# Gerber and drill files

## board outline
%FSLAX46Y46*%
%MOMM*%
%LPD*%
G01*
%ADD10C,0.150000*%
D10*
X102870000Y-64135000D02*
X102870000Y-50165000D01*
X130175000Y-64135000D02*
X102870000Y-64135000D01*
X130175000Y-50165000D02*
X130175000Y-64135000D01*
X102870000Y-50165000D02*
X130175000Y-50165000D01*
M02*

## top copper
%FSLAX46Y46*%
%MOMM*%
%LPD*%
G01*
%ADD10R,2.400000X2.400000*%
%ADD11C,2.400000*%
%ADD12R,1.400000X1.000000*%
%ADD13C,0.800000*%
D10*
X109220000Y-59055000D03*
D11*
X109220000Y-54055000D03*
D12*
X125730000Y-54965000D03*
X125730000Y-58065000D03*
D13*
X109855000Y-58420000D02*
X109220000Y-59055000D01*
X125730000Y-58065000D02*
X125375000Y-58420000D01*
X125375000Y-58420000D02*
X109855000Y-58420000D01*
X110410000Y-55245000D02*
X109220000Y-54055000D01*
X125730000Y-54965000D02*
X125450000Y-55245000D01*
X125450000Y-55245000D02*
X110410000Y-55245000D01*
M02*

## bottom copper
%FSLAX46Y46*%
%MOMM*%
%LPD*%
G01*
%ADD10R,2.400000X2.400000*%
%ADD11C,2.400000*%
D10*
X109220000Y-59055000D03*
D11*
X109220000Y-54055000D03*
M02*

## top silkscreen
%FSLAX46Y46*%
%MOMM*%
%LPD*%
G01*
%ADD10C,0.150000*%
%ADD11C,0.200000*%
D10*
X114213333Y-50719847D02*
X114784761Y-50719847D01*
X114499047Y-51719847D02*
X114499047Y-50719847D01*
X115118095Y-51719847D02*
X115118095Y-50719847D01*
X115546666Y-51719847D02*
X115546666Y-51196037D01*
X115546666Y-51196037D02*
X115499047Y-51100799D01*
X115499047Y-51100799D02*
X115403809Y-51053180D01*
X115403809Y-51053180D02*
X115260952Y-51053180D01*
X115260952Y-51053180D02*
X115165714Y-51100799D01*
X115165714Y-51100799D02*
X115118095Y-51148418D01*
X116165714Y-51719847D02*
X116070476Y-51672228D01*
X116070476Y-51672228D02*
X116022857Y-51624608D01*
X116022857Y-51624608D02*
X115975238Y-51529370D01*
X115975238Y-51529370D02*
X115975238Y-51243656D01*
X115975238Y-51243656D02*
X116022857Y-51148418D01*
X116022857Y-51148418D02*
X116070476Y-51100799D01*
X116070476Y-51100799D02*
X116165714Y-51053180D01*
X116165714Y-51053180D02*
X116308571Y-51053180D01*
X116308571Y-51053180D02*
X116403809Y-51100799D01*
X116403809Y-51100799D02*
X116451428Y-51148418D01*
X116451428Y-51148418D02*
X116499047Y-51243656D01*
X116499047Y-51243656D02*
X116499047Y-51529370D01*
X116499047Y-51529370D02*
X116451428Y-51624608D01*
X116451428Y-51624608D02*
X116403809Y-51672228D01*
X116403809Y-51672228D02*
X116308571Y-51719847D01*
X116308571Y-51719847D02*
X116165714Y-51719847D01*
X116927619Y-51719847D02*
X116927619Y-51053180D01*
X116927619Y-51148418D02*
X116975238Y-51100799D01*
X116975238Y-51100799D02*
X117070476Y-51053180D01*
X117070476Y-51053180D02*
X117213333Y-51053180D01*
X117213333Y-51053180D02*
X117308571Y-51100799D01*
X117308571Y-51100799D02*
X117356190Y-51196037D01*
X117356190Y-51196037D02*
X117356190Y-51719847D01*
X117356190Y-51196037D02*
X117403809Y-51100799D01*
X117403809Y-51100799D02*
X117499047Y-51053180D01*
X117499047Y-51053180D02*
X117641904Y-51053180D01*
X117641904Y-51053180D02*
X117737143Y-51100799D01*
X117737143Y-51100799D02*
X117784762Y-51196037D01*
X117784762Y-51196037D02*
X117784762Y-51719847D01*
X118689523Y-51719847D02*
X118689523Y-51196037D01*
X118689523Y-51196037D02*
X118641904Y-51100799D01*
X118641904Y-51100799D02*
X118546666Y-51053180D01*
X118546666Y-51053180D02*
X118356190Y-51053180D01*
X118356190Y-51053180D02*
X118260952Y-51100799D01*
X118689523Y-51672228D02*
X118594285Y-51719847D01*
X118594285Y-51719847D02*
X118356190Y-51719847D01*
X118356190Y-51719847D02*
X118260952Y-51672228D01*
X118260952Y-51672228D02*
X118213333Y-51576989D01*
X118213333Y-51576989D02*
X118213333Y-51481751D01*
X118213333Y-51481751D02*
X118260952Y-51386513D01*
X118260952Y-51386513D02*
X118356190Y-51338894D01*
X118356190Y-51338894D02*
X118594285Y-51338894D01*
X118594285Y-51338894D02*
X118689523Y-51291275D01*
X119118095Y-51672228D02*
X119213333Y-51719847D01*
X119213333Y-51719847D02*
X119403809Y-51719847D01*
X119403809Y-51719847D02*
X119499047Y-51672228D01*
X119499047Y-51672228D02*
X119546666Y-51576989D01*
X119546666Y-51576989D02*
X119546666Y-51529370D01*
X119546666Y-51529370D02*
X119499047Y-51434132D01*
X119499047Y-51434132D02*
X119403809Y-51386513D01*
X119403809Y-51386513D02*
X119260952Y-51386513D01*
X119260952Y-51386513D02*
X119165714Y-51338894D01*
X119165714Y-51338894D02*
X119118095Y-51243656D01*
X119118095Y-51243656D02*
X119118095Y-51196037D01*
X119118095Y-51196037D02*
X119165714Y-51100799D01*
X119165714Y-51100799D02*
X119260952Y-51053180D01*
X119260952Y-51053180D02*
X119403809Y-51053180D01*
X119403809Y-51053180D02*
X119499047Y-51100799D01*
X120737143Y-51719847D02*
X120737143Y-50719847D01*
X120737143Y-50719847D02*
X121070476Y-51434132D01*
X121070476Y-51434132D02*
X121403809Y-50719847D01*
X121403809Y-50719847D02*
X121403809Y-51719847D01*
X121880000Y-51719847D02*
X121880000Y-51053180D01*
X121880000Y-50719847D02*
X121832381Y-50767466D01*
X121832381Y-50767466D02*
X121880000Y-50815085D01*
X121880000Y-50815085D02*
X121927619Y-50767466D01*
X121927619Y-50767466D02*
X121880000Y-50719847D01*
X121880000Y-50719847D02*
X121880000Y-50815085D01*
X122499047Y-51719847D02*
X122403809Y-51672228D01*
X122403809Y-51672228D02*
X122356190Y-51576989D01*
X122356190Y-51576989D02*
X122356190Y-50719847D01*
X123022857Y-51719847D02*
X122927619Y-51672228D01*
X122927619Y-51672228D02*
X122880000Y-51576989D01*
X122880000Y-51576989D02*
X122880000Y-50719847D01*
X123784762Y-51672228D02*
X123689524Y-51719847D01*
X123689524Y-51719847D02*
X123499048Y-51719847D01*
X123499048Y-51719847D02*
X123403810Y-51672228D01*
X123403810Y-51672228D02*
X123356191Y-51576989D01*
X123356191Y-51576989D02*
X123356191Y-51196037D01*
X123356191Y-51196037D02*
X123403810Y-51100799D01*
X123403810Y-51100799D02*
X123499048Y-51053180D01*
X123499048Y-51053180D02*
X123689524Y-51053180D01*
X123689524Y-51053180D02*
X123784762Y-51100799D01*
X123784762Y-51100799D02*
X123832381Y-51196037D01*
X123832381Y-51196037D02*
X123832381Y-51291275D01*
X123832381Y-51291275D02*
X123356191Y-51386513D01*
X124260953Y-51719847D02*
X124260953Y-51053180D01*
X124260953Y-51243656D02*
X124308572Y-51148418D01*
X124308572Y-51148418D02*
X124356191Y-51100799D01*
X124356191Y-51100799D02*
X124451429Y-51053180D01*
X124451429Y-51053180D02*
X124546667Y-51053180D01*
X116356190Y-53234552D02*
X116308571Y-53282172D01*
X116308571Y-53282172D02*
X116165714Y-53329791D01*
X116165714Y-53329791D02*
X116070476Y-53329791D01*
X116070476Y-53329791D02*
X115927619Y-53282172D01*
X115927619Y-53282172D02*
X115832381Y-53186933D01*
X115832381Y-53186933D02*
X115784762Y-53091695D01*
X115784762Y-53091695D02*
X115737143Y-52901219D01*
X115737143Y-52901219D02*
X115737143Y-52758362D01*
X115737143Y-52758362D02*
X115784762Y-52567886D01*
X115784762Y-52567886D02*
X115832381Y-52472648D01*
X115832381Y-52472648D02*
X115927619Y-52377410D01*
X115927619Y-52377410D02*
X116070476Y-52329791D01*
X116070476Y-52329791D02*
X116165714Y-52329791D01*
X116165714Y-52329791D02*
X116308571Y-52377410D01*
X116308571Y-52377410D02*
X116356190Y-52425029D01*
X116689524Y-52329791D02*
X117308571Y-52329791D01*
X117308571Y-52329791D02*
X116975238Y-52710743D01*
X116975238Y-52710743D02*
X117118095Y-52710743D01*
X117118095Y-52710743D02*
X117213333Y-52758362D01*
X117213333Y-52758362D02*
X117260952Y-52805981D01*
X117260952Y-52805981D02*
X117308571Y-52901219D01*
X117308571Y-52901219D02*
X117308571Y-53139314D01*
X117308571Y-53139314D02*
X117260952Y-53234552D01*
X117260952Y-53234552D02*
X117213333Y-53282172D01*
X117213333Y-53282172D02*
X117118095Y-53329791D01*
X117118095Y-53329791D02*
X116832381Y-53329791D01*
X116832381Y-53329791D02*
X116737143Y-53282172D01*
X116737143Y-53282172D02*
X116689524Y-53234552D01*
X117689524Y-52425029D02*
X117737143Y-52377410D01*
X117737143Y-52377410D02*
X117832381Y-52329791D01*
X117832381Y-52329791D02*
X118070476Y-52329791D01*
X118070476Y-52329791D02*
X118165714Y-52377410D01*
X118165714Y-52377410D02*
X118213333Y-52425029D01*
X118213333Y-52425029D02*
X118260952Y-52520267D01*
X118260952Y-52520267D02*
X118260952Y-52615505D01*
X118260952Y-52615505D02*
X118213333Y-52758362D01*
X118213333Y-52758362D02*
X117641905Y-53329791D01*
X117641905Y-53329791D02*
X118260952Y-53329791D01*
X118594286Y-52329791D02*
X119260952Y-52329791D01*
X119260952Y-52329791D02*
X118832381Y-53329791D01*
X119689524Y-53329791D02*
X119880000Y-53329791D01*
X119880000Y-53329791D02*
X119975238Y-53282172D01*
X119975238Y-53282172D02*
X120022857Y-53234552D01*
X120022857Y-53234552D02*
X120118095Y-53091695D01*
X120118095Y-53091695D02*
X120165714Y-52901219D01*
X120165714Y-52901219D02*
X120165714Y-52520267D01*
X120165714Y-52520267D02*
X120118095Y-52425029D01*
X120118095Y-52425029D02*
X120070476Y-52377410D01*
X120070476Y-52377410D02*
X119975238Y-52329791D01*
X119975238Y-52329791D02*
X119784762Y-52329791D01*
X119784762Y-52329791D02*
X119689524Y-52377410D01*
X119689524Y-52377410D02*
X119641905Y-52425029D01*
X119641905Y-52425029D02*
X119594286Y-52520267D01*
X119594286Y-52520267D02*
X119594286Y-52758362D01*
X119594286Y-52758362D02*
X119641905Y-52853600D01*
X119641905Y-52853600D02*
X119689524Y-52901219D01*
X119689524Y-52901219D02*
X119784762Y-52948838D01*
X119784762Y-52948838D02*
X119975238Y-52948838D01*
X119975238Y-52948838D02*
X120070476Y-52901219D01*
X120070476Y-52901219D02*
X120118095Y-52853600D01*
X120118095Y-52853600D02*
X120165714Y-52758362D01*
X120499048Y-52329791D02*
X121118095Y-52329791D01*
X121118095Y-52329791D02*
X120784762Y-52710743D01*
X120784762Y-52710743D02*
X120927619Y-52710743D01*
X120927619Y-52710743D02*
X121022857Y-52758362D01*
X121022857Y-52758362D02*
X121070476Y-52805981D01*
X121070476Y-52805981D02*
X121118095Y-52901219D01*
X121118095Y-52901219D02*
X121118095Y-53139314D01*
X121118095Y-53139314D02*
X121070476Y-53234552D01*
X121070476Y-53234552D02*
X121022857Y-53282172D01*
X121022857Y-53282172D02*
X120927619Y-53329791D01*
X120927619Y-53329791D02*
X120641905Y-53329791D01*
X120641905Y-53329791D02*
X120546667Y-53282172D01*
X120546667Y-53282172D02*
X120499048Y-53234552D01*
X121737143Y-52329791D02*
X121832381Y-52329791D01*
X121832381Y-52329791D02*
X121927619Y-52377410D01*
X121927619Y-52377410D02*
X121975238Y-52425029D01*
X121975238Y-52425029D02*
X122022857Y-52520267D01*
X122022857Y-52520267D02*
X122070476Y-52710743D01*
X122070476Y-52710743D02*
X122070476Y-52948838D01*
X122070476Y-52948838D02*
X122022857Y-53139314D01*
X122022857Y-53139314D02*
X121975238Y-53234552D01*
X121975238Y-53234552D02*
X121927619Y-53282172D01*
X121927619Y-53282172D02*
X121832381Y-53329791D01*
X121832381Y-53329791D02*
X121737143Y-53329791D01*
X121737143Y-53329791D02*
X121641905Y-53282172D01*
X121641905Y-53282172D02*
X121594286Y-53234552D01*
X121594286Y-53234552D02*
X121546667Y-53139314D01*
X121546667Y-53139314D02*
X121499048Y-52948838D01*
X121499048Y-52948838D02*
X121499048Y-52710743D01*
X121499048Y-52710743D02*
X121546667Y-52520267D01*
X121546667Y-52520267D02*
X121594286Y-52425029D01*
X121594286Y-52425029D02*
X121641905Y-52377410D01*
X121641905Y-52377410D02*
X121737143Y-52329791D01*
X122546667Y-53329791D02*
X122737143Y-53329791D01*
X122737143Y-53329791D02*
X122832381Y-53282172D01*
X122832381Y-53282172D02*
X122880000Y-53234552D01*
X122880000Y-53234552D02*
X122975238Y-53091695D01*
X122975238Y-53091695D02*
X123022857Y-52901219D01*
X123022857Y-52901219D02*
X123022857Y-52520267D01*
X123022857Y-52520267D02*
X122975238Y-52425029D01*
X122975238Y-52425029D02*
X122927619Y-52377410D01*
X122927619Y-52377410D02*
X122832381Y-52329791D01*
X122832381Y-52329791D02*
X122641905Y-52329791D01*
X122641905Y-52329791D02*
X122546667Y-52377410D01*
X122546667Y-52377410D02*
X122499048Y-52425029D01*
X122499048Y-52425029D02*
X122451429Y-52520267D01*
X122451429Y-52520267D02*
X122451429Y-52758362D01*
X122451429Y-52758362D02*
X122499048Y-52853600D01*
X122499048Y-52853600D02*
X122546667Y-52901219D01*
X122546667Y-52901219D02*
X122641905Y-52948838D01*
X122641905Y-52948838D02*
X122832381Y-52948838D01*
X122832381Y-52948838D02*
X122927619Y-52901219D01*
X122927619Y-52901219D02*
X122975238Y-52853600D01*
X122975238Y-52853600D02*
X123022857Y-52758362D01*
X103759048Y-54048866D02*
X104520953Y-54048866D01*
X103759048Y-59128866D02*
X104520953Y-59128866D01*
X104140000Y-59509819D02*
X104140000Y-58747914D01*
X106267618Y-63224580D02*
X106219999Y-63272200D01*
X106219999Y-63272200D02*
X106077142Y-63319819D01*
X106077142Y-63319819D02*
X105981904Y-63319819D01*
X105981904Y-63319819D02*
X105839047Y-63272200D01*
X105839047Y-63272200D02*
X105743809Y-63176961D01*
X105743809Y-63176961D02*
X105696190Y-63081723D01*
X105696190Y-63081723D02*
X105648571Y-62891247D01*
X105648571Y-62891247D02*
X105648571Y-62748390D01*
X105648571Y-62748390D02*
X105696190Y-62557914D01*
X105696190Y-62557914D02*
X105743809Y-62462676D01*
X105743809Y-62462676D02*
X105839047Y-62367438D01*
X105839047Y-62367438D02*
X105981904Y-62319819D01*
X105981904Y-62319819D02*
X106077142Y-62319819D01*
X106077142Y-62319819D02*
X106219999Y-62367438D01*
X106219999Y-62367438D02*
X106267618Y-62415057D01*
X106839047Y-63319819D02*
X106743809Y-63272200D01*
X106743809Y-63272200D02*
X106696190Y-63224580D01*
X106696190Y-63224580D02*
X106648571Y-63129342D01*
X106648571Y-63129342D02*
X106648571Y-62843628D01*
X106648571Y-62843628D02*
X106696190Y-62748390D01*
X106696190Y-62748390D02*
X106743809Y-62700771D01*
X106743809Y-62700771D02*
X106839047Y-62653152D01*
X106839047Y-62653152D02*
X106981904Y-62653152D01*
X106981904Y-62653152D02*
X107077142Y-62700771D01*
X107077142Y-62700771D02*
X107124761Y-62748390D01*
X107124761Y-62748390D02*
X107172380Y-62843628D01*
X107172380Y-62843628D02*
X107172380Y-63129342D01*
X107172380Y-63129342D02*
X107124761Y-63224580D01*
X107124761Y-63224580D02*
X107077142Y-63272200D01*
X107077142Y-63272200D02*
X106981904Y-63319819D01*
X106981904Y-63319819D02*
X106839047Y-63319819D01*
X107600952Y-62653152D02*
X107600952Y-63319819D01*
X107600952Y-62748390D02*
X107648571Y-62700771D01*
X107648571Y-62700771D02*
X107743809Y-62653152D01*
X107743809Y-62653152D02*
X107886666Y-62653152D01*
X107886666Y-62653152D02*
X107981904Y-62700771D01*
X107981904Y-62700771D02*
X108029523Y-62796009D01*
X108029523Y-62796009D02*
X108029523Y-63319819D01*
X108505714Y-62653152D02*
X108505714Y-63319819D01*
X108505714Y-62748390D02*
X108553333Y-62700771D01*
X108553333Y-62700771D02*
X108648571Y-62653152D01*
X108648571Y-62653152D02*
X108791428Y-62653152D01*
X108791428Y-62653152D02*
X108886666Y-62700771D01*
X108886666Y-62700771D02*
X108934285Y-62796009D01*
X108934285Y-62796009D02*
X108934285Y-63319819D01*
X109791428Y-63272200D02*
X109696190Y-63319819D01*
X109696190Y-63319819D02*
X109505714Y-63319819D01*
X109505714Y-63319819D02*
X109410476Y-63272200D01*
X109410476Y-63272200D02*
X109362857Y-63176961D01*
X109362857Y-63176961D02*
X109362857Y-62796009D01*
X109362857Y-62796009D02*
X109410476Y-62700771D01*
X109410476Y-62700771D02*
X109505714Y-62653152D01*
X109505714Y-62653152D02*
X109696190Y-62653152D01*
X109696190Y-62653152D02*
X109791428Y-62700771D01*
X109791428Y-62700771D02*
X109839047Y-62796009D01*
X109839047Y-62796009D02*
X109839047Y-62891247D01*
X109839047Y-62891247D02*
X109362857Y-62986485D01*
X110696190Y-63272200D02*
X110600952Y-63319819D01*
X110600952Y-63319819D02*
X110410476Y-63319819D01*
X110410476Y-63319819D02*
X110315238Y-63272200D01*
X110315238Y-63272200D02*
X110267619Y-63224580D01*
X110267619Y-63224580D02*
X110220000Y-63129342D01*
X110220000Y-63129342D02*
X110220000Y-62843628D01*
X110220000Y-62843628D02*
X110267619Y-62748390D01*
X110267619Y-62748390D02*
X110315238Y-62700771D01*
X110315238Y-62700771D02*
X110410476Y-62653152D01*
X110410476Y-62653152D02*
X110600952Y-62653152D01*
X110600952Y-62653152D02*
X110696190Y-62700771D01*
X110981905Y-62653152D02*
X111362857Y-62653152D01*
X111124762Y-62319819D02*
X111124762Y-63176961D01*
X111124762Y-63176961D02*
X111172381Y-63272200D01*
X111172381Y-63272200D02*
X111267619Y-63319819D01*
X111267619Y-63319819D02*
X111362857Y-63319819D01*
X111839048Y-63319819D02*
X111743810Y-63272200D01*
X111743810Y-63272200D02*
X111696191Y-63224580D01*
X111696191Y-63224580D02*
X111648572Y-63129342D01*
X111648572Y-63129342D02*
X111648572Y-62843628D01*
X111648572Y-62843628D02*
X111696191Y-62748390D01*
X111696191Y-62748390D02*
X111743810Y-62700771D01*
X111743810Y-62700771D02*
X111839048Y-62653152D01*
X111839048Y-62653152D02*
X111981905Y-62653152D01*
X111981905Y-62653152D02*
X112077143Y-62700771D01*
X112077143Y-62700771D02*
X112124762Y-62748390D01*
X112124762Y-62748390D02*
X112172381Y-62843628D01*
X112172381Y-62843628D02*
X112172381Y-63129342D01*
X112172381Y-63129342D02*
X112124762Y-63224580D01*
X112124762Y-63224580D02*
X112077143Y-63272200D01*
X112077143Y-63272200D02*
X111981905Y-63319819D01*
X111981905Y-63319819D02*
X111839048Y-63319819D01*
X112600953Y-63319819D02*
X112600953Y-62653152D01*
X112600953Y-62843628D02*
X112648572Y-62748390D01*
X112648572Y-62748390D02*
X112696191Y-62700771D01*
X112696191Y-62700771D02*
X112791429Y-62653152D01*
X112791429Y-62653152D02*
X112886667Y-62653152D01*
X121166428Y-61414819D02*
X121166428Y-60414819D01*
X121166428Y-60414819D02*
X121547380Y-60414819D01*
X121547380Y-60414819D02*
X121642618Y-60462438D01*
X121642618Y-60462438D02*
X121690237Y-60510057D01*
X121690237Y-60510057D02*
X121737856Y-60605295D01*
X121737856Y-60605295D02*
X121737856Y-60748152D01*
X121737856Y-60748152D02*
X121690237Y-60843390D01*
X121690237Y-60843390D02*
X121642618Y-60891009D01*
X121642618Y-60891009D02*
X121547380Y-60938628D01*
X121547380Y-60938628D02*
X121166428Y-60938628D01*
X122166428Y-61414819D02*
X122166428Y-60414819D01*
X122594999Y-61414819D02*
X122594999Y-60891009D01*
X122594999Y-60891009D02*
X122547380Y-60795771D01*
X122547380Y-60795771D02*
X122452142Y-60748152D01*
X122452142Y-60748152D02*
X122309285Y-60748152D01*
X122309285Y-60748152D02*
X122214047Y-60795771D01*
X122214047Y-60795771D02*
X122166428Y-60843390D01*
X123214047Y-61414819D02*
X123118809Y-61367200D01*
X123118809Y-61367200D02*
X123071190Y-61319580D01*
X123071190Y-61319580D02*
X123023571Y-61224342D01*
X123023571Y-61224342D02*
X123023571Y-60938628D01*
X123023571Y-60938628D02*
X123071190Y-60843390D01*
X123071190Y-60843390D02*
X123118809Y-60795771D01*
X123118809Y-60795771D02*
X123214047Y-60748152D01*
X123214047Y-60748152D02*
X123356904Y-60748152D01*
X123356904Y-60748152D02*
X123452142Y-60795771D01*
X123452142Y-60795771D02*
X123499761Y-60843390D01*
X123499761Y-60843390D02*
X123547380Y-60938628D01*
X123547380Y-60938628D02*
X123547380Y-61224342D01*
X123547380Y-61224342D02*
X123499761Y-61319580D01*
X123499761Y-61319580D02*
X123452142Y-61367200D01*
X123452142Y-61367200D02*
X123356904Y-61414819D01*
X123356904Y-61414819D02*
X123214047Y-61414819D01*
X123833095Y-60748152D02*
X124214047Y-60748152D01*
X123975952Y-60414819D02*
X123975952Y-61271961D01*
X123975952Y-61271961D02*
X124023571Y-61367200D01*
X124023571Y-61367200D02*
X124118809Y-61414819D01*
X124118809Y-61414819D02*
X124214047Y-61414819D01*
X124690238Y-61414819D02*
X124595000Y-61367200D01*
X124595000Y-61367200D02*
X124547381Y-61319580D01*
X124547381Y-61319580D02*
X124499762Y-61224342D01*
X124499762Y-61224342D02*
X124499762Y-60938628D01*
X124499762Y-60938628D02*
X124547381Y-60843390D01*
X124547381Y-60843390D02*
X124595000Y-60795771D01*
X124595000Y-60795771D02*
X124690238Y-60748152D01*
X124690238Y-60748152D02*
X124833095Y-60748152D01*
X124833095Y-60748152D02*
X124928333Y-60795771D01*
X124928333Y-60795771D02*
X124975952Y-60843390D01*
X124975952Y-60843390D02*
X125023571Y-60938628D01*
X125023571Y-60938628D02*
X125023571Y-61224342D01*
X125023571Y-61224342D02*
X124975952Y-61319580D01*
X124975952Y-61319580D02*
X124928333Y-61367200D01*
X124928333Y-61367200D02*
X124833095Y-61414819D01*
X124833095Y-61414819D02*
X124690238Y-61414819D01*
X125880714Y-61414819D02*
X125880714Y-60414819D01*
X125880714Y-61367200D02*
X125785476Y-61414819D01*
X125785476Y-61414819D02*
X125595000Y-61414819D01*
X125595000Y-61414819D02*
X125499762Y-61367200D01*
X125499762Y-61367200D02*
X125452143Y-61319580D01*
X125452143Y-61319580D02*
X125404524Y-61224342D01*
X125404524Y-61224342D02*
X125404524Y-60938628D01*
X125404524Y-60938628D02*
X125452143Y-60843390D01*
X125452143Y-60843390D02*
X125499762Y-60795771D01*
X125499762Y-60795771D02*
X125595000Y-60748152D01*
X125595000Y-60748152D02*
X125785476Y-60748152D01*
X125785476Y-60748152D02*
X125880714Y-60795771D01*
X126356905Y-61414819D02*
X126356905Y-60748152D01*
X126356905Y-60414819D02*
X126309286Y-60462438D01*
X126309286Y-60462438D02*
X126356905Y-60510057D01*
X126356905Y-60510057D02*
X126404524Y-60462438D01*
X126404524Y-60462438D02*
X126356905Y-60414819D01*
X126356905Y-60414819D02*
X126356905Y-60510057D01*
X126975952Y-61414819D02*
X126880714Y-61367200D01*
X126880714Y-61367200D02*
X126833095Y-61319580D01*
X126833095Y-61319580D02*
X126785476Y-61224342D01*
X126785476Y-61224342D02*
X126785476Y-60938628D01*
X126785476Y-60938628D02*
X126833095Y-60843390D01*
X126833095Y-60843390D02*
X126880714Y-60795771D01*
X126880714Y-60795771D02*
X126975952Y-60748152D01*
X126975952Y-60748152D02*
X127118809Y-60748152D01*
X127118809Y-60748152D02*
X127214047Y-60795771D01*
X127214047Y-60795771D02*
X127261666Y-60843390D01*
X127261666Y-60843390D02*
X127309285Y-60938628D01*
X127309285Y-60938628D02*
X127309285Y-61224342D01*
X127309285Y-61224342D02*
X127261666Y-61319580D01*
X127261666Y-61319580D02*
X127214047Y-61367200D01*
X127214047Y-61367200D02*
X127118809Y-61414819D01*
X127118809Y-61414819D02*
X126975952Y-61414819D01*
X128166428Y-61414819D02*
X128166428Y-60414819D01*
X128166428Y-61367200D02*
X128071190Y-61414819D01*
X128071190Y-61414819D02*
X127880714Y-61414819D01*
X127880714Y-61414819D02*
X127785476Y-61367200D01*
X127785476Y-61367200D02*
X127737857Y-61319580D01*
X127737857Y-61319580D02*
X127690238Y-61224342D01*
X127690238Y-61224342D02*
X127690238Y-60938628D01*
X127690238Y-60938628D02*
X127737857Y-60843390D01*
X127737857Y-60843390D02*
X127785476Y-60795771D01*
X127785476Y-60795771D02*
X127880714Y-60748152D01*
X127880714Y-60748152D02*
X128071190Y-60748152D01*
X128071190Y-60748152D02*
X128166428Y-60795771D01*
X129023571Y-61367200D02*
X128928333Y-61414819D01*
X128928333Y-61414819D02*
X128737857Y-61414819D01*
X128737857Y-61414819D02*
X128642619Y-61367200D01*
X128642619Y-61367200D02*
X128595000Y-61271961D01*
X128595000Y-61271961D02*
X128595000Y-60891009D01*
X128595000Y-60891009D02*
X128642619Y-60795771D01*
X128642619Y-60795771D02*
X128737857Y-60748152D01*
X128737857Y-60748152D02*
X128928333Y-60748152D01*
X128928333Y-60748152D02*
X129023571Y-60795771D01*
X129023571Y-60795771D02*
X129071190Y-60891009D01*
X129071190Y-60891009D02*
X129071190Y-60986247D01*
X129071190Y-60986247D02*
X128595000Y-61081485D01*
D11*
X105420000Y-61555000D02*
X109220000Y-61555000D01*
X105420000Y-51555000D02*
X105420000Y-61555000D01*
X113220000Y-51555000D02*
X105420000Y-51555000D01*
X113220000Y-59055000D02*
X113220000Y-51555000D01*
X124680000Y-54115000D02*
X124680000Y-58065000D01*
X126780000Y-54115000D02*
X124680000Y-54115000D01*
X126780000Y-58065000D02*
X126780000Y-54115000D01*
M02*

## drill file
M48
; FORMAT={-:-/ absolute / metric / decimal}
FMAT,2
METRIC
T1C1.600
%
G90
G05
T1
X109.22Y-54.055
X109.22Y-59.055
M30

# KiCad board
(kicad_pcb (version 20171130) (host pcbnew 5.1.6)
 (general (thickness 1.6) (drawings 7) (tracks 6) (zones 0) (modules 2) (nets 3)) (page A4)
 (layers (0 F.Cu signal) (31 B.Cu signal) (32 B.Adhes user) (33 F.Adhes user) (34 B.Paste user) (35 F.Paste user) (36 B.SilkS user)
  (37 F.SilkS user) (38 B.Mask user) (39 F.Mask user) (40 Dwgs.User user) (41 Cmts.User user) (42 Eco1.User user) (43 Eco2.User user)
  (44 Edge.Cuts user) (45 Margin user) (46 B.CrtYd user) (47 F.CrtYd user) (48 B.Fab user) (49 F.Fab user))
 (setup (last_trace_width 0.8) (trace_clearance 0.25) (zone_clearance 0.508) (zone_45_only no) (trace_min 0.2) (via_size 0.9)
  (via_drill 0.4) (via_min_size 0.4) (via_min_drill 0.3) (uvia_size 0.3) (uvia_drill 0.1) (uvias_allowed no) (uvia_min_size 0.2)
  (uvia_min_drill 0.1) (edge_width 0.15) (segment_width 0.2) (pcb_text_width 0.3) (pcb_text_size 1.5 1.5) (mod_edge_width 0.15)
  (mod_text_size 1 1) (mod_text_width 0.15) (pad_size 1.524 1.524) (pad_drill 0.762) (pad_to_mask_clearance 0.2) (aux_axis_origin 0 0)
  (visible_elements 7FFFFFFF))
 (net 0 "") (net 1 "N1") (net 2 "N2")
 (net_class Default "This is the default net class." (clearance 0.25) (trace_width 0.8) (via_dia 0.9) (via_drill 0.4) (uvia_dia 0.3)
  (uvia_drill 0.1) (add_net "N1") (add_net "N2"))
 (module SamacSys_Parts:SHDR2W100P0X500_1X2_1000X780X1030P (layer F.Cu) (at 109.22 59.055 90)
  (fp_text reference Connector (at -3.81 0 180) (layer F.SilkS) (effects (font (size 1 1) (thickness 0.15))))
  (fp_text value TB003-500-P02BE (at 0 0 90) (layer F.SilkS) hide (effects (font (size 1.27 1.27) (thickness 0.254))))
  (fp_line (start -2.5 -3.8) (end -2.5 0) (layer F.SilkS) (width 0.2))
  (fp_line (start 7.5 -3.8) (end -2.5 -3.8) (layer F.SilkS) (width 0.2))
  (fp_line (start 7.5 4) (end 7.5 -3.8) (layer F.SilkS) (width 0.2))
  (fp_line (start 0 4) (end 7.5 4) (layer F.SilkS) (width 0.2))
  (pad 1 thru_hole rect (at 0 0 90) (size 2.4 2.4) (drill 1.6) (layers *.Cu *.Mask) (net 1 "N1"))
  (pad 2 thru_hole circle (at 5 0 90) (size 2.4 2.4) (drill 1.6) (layers *.Cu *.Mask) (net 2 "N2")))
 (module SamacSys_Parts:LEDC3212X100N (layer F.Cu) (at 125.73 56.515 270)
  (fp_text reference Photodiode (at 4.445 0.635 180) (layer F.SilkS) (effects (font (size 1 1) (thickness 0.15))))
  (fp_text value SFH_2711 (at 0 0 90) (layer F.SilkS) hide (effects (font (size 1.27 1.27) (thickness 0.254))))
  (fp_line (start -2.4 1.05) (end 1.55 1.05) (layer F.SilkS) (width 0.2))
  (fp_line (start -2.4 -1.05) (end -2.4 1.05) (layer F.SilkS) (width 0.2))
  (fp_line (start 1.55 -1.05) (end -2.4 -1.05) (layer F.SilkS) (width 0.2))
  (pad 1 smd rect (at -1.55 0 270) (size 1 1.4) (layers F.Cu F.Paste F.Mask) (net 2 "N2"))
  (pad 2 smd rect (at 1.55 0 270) (size 1 1.4) (layers F.Cu F.Paste F.Mask) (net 1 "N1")))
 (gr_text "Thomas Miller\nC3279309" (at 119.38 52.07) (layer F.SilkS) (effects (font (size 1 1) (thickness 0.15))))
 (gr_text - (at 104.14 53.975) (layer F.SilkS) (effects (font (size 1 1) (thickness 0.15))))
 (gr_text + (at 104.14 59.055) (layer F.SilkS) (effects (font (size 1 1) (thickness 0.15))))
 (gr_line (start 102.87 64.135) (end 102.87 50.165) (layer Edge.Cuts) (width 0.15))
 (gr_line (start 130.175 64.135) (end 102.87 64.135) (layer Edge.Cuts) (width 0.15))
 (gr_line (start 130.175 50.165) (end 130.175 64.135) (layer Edge.Cuts) (width 0.15))
 (gr_line (start 102.87 50.165) (end 130.175 50.165) (layer Edge.Cuts) (width 0.15))
 (segment (start 109.855 58.42) (end 109.22 59.055) (width 0.8) (layer F.Cu) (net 1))
 (segment (start 125.73 58.065) (end 125.375 58.42) (width 0.8) (layer F.Cu) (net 1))
 (segment (start 125.375 58.42) (end 109.855 58.42) (width 0.8) (layer F.Cu) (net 1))
 (segment (start 110.41 55.245) (end 109.22 54.055) (width 0.8) (layer F.Cu) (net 2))
 (segment (start 125.73 54.965) (end 125.45 55.245) (width 0.8) (layer F.Cu) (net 2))
 (segment (start 125.45 55.245) (end 110.41 55.245) (width 0.8) (layer F.Cu) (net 2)))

